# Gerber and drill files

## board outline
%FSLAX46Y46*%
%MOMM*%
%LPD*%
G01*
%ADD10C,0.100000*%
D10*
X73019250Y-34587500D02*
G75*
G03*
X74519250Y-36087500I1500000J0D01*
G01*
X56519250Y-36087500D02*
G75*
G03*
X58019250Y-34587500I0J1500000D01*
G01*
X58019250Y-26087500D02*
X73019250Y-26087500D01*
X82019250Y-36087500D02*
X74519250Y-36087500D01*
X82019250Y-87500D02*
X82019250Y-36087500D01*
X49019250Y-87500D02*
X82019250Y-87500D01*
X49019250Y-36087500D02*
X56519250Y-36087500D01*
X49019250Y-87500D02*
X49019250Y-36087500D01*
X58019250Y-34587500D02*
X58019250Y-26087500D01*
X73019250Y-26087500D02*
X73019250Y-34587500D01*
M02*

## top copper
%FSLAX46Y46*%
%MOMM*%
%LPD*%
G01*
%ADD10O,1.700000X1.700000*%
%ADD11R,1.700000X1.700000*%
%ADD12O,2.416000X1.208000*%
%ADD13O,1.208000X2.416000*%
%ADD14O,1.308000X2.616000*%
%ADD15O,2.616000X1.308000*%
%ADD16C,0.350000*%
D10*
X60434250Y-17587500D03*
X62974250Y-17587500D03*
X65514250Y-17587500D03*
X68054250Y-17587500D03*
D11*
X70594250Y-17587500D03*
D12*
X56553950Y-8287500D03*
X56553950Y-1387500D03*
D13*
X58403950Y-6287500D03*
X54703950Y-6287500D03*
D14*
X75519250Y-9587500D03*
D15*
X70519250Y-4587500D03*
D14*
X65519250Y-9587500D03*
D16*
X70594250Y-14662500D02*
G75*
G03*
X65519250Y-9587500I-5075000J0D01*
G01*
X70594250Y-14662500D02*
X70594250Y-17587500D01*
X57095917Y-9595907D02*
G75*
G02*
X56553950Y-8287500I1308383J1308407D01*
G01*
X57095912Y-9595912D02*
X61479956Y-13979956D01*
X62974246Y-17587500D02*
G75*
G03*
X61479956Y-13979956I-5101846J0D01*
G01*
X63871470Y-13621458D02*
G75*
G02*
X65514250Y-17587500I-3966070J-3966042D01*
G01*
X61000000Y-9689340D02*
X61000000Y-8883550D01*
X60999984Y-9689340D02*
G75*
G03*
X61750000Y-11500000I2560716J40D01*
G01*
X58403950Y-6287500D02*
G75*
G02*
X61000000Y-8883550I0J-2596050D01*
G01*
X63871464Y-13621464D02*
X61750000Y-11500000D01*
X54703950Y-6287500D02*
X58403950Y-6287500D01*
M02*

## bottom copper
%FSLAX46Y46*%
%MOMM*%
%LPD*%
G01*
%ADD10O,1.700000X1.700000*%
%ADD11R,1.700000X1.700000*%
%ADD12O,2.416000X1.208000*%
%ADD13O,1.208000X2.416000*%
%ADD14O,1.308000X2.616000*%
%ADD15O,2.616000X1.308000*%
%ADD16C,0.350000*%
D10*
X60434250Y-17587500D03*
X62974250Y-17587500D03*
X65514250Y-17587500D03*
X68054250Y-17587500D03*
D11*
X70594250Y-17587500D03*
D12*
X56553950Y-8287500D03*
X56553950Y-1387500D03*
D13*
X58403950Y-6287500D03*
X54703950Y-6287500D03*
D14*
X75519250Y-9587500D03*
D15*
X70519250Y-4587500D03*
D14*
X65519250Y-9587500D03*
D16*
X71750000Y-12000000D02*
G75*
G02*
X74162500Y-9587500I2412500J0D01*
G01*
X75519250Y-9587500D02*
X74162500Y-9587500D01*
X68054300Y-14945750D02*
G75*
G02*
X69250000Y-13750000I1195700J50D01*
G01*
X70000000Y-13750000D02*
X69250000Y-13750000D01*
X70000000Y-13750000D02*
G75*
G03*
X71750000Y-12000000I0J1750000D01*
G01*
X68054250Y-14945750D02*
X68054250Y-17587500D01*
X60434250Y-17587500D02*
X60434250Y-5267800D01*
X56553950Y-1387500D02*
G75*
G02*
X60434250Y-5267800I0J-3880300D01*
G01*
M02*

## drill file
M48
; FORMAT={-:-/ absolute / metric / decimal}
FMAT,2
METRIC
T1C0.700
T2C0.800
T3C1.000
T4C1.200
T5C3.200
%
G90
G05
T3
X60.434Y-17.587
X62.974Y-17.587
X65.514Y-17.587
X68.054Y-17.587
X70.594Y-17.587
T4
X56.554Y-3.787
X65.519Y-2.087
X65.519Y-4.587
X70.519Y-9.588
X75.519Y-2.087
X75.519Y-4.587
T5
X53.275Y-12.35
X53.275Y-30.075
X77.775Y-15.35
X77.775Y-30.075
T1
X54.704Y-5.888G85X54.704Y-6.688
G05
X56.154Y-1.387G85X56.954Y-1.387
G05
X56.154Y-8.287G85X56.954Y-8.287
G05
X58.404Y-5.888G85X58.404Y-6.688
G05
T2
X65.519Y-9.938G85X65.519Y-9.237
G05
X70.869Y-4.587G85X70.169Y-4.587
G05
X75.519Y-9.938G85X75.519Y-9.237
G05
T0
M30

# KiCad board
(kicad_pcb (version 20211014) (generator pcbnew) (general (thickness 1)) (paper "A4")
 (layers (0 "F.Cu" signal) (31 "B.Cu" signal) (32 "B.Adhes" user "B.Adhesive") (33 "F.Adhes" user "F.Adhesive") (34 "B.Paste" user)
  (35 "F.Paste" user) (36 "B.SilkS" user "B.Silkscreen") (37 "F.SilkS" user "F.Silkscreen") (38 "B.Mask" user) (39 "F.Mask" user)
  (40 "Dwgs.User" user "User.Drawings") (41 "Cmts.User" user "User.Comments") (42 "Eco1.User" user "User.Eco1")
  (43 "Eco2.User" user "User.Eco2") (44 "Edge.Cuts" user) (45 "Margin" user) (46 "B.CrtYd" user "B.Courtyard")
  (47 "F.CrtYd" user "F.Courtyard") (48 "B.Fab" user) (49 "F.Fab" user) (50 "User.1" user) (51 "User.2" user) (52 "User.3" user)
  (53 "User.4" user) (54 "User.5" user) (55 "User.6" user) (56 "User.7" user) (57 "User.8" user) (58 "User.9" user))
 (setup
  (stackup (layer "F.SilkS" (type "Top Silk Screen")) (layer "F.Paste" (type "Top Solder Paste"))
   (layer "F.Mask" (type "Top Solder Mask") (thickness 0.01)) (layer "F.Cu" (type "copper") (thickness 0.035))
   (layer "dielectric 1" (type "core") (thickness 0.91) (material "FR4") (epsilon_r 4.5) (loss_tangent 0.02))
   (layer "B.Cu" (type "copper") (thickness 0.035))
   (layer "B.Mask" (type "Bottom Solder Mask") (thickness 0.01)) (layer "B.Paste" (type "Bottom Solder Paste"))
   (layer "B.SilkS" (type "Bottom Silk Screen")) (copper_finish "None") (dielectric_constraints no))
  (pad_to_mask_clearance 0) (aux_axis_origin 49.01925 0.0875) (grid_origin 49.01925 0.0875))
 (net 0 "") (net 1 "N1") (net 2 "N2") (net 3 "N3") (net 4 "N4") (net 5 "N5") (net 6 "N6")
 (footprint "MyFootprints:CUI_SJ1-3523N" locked (layer "F.Cu") (at 70.51925 4.5875 180)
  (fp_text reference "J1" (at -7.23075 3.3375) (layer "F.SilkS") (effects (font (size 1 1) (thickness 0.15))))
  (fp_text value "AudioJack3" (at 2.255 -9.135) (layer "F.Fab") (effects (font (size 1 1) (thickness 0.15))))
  (pad "" np_thru_hole circle locked (at 0 -5 180) (size 1.2 1.2) (drill 1.2) (layers *.Cu *.Mask))
  (pad "" np_thru_hole circle locked (at 5 0 180) (size 1.2 1.2) (drill 1.2) (layers *.Cu *.Mask))
  (pad "" np_thru_hole circle locked (at -5 2.5 180) (size 1.2 1.2) (drill 1.2) (layers *.Cu *.Mask))
  (pad "" np_thru_hole circle locked (at 5 2.5 180) (size 1.2 1.2) (drill 1.2) (layers *.Cu *.Mask))
  (pad "" np_thru_hole circle locked (at -5 0 180) (size 1.2 1.2) (drill 1.2) (layers *.Cu *.Mask))
  (pad "R" thru_hole oval locked (at -5 -5 180) (size 1.308 2.616) (drill oval 0.8 1.5) (layers *.Cu *.Mask) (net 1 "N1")
   (solder_mask_margin 0.102))
  (pad "S" thru_hole oval locked (at 0 0 180) (size 2.616 1.308) (drill oval 1.5 0.8) (layers *.Cu *.Mask) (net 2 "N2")
   (solder_mask_margin 0.102))
  (pad "T" thru_hole oval locked (at 5 -5 180) (size 1.308 2.616) (drill oval 0.8 1.5) (layers *.Cu *.Mask) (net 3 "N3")
   (solder_mask_margin 0.102)))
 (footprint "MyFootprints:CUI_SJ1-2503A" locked (layer "F.Cu") (at 56.55395 1.3875)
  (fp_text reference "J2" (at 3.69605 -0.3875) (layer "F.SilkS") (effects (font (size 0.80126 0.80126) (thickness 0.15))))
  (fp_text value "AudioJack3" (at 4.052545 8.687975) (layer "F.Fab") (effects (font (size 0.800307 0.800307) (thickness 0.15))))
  (pad "" np_thru_hole circle locked (at 0 2.4) (size 1.2 1.2) (drill 1.2) (layers *.Cu *.Mask))
  (pad "R" thru_hole oval locked (at 0 6.9) (size 2.416 1.208) (drill oval 1.5 0.7) (layers *.Cu *.Mask) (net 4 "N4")
   (solder_mask_margin 0.102))
  (pad "S" thru_hole oval locked (at 0 0) (size 2.416 1.208) (drill oval 1.5 0.7) (layers *.Cu *.Mask) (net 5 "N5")
   (solder_mask_margin 0.102))
  (pad "T" thru_hole oval locked (at 1.85 4.9) (size 1.208 2.416) (drill oval 0.7 1.5) (layers *.Cu *.Mask) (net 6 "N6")
   (solder_mask_margin 0.102))
  (pad "T" thru_hole oval locked (at -1.85 4.9) (size 1.208 2.416) (drill oval 0.7 1.5) (layers *.Cu *.Mask) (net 6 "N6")
   (solder_mask_margin 0.102)))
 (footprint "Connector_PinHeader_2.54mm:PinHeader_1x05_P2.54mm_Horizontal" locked (layer "F.Cu") (at 70.59425 17.5875 -90)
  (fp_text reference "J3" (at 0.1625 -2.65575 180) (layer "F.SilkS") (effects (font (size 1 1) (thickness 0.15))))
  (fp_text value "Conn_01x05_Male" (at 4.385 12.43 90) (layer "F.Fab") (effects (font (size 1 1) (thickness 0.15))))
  (pad "1" thru_hole rect locked (at 0 0 270) (size 1.7 1.7) (drill 1) (layers *.Cu *.Mask) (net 3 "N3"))
  (pad "2" thru_hole oval locked (at 0 2.54 270) (size 1.7 1.7) (drill 1) (layers *.Cu *.Mask) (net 1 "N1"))
  (pad "3" thru_hole oval locked (at 0 5.08 270) (size 1.7 1.7) (drill 1) (layers *.Cu *.Mask) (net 6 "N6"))
  (pad "4" thru_hole oval locked (at 0 7.62 270) (size 1.7 1.7) (drill 1) (layers *.Cu *.Mask) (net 4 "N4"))
  (pad "5" thru_hole oval locked (at 0 10.16 270) (size 1.7 1.7) (drill 1) (layers *.Cu *.Mask) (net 5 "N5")))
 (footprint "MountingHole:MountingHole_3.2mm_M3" (layer "F.Cu") (at 77.775 30.075)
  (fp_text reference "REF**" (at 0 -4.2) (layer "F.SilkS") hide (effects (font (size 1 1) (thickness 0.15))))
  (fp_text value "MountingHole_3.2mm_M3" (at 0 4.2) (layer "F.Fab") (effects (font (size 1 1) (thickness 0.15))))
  (pad "" np_thru_hole circle locked (at 0 0) (size 3.2 3.2) (drill 3.2) (layers *.Cu *.Mask)))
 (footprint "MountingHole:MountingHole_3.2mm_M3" (layer "F.Cu") (at 53.275 12.35)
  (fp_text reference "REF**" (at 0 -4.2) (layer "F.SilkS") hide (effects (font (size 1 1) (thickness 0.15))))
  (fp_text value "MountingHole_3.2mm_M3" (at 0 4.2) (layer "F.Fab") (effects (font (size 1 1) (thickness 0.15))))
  (pad "" np_thru_hole circle locked (at 0 0) (size 3.2 3.2) (drill 3.2) (layers *.Cu *.Mask)))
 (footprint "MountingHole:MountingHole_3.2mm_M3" (layer "F.Cu") (at 77.775 15.35)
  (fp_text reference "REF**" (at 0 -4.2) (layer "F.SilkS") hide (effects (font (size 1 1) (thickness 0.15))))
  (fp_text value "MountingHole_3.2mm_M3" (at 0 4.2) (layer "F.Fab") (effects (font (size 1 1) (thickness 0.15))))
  (pad "" np_thru_hole circle locked (at 0 0) (size 3.2 3.2) (drill 3.2) (layers *.Cu *.Mask)))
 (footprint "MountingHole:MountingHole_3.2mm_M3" (layer "F.Cu") (at 53.275 30.075)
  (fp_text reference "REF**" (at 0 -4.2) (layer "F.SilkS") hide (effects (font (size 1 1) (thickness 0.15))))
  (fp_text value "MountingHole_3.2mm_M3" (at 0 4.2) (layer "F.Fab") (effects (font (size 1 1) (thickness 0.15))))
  (pad "" np_thru_hole circle locked (at 0 0) (size 3.2 3.2) (drill 3.2) (layers *.Cu *.Mask)))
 (gr_line (start 49.01925 0.0875) (end 82.01925 0.0875) (layer "Edge.Cuts") (width 0.1))
 (gr_arc (start 58.01925 34.5875) (mid 57.57991 35.64816) (end 56.51925 36.0875) (layer "Edge.Cuts") (width 0.1))
 (gr_line (start 82.01925 36.0875) (end 74.51925 36.0875) (layer "Edge.Cuts") (width 0.1))
 (gr_arc (start 74.51925 36.0875) (mid 73.45859 35.64816) (end 73.01925 34.5875) (layer "Edge.Cuts") (width 0.1))
 (gr_line (start 49.01925 36.0875) (end 56.51925 36.0875) (layer "Edge.Cuts") (width 0.1))
 (gr_line (start 82.01925 0.0875) (end 82.01925 36.0875) (layer "Edge.Cuts") (width 0.1))
 (gr_line (start 49.01925 0.0875) (end 49.01925 36.0875) (layer "Edge.Cuts") (width 0.1))
 (gr_line (start 73.01925 26.0875) (end 73.01925 34.5875) (layer "Edge.Cuts") (width 0.1))
 (gr_line (start 58.01925 34.5875) (end 58.01925 26.0875) (layer "Edge.Cuts") (width 0.1))
 (gr_line (start 58.01925 26.0875) (end 73.01925 26.0875) (layer "Edge.Cuts") (width 0.1))
 (segment (start 68.05425 14.94575) (end 68.05425 17.5875) (width 0.35) (layer "B.Cu") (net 1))
 (segment (start 70 13.75) (end 69.25 13.75) (width 0.35) (layer "B.Cu") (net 1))
 (segment (start 75.51925 9.5875) (end 74.1625 9.5875) (width 0.35) (layer "B.Cu") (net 1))
 (arc (start 71.75 12) (mid 71.237437 13.237437) (end 70 13.75) (width 0.35) (layer "B.Cu") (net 1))
 (arc (start 69.25 13.75) (mid 68.404477 14.100227) (end 68.05425 14.94575) (width 0.35) (layer "B.Cu") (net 1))
 (arc (start 74.1625 9.5875) (mid 72.456605 10.294105) (end 71.75 12) (width 0.35) (layer "B.Cu") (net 1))
 (segment (start 70.59425 14.6625) (end 70.59425 17.5875) (width 0.35) (layer "F.Cu") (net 3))
 (arc (start 65.51925 9.5875) (mid 69.107817 11.073933) (end 70.59425 14.6625) (width 0.35) (layer "F.Cu") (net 3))
 (segment (start 57.095912 9.595912) (end 61.479956 13.979956) (width 0.35) (layer "F.Cu") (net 4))
 (arc (start 61.479956 13.979956) (mid 62.585895 15.635111) (end 62.97425 17.5875) (width 0.35) (layer "F.Cu") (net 4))
 (arc (start 56.55395 8.2875) (mid 56.694801 8.995607) (end 57.095912 9.595912) (width 0.35) (layer "F.Cu") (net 4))
 (segment (start 60.43425 17.5875) (end 60.43425 5.2678) (width 0.35) (layer "B.Cu") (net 5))
 (arc (start 60.43425 5.2678) (mid 59.297736 2.524014) (end 56.55395 1.3875) (width 0.35) (layer "B.Cu") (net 5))
 (segment (start 61 9.68934) (end 61 8.88355) (width 0.35) (layer "F.Cu") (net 6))
 (segment (start 54.70395 6.2875) (end 58.40395 6.2875) (width 0.35) (layer "F.Cu") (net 6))
 (segment (start 63.871464 13.621464) (end 61.75 11.5) (width 0.35) (layer "F.Cu") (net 6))
 (arc (start 61.75 11.5) (mid 61.194918 10.669262) (end 61 9.68934) (width 0.35) (layer "F.Cu") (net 6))
 (arc (start 65.51425 17.5875) (mid 65.087304 15.441097) (end 63.871464 13.621464) (width 0.35) (layer "F.Cu") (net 6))
 (arc (start 61 8.88355) (mid 60.239635 7.047865) (end 58.40395 6.2875) (width 0.35) (layer "F.Cu") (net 6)))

